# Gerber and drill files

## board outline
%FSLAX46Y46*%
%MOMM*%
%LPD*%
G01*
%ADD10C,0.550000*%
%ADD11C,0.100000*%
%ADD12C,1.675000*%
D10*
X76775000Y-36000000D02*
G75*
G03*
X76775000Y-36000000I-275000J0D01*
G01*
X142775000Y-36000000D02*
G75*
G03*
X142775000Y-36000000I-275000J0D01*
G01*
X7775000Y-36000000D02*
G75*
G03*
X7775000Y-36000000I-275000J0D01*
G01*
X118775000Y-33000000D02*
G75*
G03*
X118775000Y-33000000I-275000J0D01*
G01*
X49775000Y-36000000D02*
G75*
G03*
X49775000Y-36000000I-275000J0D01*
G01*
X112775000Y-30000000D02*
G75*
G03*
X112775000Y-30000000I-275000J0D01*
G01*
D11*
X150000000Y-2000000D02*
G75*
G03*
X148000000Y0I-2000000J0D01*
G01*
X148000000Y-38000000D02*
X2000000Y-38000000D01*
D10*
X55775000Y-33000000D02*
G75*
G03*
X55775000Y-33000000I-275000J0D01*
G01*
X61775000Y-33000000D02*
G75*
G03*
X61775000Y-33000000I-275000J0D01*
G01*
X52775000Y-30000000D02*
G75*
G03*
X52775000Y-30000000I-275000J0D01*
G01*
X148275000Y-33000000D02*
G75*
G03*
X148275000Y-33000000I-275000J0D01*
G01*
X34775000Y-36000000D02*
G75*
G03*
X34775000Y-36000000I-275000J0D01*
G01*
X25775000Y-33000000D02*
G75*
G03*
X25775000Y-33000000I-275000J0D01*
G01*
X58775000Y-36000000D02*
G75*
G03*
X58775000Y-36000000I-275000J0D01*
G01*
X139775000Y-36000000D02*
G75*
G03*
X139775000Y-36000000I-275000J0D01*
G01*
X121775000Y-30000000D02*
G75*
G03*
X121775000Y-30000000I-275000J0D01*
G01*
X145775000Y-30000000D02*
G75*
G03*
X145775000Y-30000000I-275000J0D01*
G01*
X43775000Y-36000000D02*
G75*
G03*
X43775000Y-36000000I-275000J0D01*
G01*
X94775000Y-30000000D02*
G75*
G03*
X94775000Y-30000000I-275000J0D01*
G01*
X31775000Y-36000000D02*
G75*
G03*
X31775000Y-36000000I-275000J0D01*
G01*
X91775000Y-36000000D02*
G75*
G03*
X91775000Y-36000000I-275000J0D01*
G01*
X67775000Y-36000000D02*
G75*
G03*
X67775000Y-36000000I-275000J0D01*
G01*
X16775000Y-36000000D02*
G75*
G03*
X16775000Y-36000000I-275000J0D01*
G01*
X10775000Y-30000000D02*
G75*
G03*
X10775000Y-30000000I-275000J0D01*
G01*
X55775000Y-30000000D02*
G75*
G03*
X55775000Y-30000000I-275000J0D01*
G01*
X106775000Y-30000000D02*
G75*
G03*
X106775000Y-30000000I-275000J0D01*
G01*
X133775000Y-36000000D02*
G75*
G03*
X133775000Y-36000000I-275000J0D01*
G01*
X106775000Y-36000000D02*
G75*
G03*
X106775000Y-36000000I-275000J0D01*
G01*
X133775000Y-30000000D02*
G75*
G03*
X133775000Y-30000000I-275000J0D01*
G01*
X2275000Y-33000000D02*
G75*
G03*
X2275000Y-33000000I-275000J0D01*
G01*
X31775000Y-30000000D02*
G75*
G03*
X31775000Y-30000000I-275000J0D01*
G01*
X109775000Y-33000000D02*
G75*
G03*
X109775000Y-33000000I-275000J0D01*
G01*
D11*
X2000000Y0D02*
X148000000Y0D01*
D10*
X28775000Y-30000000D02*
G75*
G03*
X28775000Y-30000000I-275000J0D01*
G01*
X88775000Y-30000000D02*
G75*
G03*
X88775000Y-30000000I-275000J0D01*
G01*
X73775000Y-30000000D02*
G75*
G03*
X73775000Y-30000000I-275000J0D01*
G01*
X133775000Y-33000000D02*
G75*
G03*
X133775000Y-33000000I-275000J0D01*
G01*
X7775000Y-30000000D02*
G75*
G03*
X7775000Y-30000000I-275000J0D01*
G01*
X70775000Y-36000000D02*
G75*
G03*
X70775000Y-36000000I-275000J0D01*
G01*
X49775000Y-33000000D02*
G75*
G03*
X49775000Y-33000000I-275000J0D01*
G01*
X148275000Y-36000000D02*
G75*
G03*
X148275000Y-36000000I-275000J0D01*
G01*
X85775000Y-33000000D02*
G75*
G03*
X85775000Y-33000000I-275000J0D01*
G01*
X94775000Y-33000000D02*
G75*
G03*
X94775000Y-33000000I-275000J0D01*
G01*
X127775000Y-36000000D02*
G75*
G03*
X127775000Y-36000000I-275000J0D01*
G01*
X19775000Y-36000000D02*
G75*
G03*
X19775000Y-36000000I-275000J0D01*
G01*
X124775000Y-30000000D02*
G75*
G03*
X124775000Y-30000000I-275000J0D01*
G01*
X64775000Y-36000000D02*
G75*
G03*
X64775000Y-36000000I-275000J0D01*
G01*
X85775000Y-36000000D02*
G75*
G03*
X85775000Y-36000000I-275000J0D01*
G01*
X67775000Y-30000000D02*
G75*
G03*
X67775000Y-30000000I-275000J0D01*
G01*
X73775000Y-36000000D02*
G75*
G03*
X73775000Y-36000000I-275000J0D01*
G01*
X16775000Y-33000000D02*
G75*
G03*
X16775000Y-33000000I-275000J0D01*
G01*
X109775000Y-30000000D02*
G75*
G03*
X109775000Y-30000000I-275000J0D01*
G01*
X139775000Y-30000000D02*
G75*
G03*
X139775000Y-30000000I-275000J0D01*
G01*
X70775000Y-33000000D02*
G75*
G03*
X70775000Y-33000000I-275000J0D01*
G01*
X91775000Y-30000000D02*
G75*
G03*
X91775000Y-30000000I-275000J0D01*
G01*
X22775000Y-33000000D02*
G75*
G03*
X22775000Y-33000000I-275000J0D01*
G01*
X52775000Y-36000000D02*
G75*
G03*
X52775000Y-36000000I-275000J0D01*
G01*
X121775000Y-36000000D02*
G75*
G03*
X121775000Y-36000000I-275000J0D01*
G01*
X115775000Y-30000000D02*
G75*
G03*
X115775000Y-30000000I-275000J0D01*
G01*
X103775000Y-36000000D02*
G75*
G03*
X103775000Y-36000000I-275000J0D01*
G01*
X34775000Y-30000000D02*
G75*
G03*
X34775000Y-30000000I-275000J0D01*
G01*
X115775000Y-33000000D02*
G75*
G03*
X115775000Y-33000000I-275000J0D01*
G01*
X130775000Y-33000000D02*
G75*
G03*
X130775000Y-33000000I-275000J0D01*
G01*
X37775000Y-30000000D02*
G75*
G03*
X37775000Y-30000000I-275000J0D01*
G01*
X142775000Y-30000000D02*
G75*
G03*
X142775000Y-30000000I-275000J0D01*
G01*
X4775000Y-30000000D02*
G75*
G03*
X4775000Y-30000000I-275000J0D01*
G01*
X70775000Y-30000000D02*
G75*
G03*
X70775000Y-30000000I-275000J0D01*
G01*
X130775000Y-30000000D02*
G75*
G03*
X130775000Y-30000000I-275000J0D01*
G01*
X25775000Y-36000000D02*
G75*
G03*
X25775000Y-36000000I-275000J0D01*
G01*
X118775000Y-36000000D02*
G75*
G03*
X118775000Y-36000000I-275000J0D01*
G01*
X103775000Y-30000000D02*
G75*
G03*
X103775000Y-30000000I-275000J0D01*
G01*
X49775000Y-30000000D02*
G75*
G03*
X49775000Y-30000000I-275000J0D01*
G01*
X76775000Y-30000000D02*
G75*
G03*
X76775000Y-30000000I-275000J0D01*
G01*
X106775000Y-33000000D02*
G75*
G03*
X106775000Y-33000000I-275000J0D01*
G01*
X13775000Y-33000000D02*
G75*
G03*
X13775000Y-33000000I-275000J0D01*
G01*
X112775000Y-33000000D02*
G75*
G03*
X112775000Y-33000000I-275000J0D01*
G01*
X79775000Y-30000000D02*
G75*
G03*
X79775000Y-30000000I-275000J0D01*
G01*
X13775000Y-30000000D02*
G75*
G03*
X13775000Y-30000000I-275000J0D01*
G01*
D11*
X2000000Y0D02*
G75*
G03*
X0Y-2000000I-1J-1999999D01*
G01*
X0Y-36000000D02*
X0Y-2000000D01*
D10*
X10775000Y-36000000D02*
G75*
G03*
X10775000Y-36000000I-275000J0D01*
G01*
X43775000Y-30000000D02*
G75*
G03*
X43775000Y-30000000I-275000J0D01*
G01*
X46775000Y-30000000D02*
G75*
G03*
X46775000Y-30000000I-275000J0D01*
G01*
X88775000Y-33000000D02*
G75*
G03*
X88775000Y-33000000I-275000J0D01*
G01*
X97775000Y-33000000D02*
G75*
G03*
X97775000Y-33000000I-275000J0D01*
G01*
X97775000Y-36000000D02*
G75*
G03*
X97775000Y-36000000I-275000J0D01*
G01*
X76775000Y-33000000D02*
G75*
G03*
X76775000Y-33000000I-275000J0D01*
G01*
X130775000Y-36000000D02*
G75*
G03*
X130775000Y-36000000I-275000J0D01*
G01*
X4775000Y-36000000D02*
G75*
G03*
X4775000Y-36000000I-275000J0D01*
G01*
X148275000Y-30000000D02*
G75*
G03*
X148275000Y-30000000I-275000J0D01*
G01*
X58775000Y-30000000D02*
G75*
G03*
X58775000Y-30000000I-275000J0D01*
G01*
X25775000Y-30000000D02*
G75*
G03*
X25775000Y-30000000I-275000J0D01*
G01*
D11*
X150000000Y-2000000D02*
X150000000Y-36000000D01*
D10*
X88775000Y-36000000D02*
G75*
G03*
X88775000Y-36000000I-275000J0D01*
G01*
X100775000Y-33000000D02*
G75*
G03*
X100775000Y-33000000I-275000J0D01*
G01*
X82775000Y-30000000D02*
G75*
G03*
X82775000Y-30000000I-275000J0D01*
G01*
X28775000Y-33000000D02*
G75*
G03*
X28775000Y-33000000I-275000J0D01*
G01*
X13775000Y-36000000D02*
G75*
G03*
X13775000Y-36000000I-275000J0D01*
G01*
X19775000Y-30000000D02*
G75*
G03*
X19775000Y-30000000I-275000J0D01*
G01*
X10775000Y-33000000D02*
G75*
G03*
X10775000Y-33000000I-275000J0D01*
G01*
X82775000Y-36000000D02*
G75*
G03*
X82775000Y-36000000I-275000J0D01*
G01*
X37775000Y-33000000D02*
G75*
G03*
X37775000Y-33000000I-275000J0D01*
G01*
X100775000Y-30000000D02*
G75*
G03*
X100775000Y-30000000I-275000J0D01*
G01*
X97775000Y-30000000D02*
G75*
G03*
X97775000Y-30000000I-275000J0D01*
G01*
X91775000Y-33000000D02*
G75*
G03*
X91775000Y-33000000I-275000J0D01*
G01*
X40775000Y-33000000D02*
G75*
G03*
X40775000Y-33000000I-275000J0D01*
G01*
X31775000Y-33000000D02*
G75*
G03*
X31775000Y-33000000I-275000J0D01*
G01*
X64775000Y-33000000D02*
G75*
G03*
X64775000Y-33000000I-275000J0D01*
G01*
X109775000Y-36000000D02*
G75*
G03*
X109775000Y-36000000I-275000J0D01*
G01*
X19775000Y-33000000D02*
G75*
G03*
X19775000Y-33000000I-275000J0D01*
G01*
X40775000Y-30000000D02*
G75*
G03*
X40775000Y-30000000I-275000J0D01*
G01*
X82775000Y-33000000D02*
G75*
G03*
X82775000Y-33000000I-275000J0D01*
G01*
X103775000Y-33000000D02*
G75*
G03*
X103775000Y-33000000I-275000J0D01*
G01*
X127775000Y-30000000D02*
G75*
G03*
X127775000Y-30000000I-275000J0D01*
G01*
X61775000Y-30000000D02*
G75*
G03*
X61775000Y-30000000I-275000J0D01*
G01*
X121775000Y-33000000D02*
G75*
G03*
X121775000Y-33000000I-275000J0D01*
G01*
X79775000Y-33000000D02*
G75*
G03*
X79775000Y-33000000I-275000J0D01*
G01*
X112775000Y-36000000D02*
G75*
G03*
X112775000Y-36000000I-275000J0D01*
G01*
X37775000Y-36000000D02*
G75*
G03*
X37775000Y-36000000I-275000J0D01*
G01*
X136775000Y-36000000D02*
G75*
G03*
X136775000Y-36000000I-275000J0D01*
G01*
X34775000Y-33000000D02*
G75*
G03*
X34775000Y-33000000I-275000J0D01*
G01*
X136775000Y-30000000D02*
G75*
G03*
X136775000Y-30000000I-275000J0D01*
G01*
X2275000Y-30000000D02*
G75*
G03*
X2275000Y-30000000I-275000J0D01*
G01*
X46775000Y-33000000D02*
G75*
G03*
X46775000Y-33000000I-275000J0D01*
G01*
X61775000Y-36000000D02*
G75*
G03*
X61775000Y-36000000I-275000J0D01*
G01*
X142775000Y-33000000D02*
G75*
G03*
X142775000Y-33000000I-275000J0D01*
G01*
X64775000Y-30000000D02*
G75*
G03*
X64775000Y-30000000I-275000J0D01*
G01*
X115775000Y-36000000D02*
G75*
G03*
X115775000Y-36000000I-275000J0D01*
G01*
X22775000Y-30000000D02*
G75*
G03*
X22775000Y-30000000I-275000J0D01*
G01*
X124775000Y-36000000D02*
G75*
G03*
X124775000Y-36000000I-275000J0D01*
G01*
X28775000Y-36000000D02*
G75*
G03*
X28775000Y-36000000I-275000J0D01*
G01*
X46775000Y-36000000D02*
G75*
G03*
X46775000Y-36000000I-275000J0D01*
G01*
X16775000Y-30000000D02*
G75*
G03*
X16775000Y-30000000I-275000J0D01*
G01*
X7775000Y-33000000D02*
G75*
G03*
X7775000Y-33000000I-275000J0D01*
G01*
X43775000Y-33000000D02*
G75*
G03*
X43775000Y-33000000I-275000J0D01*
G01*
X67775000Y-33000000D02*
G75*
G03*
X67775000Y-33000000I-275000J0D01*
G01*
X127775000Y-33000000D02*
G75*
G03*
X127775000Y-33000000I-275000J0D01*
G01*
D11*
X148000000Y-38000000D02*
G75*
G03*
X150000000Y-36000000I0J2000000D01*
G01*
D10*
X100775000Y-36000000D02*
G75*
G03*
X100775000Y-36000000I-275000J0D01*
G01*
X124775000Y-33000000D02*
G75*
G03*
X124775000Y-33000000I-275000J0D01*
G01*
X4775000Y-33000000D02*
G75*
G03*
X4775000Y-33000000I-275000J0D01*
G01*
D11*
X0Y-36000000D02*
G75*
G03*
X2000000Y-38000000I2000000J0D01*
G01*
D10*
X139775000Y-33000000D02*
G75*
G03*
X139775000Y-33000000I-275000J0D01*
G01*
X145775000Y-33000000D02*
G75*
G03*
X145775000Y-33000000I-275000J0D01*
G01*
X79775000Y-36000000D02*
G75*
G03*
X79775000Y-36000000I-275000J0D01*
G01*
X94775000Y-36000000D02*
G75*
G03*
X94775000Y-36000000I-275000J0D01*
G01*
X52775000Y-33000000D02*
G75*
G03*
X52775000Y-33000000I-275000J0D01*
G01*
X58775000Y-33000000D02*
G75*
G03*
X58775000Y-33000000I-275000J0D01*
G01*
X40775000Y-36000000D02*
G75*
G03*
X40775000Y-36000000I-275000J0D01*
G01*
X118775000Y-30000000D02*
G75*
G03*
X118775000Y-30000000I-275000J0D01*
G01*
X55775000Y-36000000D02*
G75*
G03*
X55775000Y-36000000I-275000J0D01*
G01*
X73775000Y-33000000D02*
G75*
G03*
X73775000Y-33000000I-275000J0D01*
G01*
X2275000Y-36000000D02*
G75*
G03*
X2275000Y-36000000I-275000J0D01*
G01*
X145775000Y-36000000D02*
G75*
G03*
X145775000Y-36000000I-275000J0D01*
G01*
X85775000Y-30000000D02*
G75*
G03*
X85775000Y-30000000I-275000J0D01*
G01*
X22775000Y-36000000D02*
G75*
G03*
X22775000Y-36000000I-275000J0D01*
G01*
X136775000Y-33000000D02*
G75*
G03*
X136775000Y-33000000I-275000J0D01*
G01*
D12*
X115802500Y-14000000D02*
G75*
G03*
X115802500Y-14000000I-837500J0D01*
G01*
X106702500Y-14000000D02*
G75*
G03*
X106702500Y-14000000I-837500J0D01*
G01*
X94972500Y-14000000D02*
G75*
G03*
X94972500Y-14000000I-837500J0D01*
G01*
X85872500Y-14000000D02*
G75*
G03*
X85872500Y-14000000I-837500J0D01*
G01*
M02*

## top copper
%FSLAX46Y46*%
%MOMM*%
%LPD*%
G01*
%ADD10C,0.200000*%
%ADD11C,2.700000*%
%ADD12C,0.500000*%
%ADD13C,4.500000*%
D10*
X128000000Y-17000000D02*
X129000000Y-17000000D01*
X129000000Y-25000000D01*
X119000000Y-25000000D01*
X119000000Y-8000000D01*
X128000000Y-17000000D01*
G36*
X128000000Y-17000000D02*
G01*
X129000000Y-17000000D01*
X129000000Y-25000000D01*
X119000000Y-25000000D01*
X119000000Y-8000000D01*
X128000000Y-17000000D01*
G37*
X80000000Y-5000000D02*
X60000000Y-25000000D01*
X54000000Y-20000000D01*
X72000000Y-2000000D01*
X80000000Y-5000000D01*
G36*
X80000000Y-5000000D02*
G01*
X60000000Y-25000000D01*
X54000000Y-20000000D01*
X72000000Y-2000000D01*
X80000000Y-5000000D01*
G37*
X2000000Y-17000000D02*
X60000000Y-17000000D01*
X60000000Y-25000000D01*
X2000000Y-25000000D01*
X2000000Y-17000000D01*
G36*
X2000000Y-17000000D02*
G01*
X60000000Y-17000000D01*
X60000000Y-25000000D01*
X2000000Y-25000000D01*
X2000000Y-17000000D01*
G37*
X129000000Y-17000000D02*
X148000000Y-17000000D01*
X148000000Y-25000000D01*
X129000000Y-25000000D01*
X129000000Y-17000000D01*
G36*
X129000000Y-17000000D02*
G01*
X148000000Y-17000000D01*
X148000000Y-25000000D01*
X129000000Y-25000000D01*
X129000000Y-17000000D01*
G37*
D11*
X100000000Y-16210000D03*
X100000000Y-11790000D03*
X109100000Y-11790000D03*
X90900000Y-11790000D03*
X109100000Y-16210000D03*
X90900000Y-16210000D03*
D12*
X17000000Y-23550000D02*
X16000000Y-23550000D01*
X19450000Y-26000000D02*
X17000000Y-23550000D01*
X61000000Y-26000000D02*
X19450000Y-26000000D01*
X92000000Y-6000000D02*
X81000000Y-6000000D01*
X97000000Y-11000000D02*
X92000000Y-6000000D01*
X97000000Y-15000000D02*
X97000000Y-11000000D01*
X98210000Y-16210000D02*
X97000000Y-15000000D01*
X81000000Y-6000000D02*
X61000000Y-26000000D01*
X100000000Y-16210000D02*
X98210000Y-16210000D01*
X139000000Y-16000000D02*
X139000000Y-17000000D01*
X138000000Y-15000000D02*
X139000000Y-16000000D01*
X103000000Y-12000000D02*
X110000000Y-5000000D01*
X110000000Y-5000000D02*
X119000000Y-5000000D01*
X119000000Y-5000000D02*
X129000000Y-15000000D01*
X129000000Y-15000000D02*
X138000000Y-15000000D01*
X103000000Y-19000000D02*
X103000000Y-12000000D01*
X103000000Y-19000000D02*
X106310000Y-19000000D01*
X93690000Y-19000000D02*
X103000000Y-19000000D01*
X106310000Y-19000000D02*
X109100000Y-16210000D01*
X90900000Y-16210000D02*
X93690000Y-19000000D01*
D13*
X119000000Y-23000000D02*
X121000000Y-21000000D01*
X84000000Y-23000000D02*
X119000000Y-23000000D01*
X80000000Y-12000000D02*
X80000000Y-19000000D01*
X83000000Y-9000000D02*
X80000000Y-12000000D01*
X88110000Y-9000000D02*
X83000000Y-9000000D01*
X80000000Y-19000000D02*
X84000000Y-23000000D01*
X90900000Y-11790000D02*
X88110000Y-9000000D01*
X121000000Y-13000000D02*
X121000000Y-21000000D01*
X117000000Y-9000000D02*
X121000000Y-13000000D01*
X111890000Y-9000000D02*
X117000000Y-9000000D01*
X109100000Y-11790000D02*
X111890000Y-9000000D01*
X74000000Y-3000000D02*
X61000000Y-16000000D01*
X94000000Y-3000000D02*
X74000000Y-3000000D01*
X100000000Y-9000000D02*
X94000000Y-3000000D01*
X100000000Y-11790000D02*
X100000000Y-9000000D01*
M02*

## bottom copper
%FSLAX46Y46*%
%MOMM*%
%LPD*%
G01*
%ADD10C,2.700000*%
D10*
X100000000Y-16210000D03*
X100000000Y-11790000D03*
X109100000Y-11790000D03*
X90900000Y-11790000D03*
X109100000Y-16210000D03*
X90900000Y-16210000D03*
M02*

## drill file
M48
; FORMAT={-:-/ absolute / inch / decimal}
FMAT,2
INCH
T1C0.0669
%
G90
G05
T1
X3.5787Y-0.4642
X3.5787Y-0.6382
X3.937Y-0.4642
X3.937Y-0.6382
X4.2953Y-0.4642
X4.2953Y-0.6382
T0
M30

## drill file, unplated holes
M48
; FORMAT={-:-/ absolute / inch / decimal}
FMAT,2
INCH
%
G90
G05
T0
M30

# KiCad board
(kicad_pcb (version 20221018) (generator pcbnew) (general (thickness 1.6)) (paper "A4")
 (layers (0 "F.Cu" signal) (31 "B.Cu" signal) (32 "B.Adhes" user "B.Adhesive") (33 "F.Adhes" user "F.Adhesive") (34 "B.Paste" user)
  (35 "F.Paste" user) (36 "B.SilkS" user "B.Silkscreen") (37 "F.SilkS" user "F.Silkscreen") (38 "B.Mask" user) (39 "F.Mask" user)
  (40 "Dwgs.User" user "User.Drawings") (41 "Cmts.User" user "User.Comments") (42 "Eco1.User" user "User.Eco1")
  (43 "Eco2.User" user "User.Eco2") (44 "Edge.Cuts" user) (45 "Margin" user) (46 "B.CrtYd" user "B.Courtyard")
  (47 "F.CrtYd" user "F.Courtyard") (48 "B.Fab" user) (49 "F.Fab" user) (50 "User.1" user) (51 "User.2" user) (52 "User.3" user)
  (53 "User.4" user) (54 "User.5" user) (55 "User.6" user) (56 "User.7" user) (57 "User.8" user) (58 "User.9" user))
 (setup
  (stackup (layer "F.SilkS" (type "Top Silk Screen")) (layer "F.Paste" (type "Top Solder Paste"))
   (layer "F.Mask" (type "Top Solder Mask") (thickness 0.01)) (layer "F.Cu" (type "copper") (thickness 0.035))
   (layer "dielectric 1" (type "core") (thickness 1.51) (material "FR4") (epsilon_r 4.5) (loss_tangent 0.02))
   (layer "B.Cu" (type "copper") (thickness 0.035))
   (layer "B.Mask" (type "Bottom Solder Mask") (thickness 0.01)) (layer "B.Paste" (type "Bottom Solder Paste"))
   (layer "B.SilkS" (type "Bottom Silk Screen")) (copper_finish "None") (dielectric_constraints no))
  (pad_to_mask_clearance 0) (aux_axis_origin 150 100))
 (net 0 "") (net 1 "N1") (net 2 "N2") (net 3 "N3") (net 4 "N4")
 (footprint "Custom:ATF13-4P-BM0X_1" (layer "F.Cu") (at 100 14 180)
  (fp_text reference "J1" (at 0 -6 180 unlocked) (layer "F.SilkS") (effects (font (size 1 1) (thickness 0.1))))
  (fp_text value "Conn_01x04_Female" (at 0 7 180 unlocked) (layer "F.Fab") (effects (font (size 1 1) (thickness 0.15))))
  (fp_circle (center -14.965 0) (end -13.315 0) (stroke (width 0.05) (type solid)) (fill solid) (layer "Edge.Cuts"))
  (fp_circle (center -5.865 0) (end -4.215 0) (stroke (width 0.05) (type solid)) (fill solid) (layer "Edge.Cuts"))
  (fp_circle (center 5.865 0) (end 7.515 0) (stroke (width 0.05) (type solid)) (fill solid) (layer "Edge.Cuts"))
  (fp_circle (center 14.965 0) (end 16.615 0) (stroke (width 0.05) (type solid)) (fill solid) (layer "Edge.Cuts"))
  (pad "1" thru_hole circle (at 0 -2.21 180) (size 2.7 2.7) (drill 1.7) (layers "*.Cu" "*.Mask") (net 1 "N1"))
  (pad "2" thru_hole circle (at 0 2.21 180) (size 2.7 2.7) (drill 1.7) (layers "*.Cu" "*.Mask") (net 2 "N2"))
  (pad "3" thru_hole circle (at -9.1 2.21 180) (size 2.7 2.7) (drill 1.7) (layers "*.Cu" "*.Mask") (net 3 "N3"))
  (pad "3" thru_hole circle (at 9.1 2.21 180) (size 2.7 2.7) (drill 1.7) (layers "*.Cu" "*.Mask") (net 3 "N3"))
  (pad "4" thru_hole circle (at -9.1 -2.21 180) (size 2.7 2.7) (drill 1.7) (layers "*.Cu" "*.Mask") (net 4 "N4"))
  (pad "4" thru_hole circle (at 9.1 -2.21 180) (size 2.7 2.7) (drill 1.7) (layers "*.Cu" "*.Mask") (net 4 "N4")))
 (gr_poly (pts (xy 60 25) (xy 80 5) (xy 72 2) (xy 54 20)) (stroke (width 0.2) (type solid)) (fill solid) (layer "F.Cu"))
 (gr_poly (pts (xy 129 25) (xy 119 25) (xy 119 8) (xy 128 17) (xy 129 17)) (stroke (width 0.2) (type solid)) (fill solid) (layer "F.Cu"))
 (gr_rect (start 2 17) (end 60 25) (stroke (width 0.2) (type solid)) (fill solid) (layer "F.Cu"))
 (gr_rect (start 129 17) (end 148 25) (stroke (width 0.2) (type solid)) (fill solid) (layer "F.Cu"))
 (gr_circle (center 76.5 36) (end 76.5 36.5) (stroke (width 0.1) (type solid)) (fill solid) (layer "Edge.Cuts"))
 (gr_circle (center 142.5 36) (end 142.5 36.5) (stroke (width 0.1) (type solid)) (fill solid) (layer "Edge.Cuts"))
 (gr_circle (center 7.5 36) (end 7.5 36.5) (stroke (width 0.1) (type solid)) (fill solid) (layer "Edge.Cuts"))
 (gr_circle (center 118.5 33) (end 118.5 33.5) (stroke (width 0.1) (type solid)) (fill solid) (layer "Edge.Cuts"))
 (gr_circle (center 49.5 36) (end 49.5 36.5) (stroke (width 0.1) (type solid)) (fill solid) (layer "Edge.Cuts"))
 (gr_circle (center 112.5 30) (end 112.5 30.5) (stroke (width 0.1) (type solid)) (fill solid) (layer "Edge.Cuts"))
 (gr_arc (start 148 0) (mid 149.414214 0.585786) (end 150 2) (stroke (width 0.1) (type default)) (layer "Edge.Cuts"))
 (gr_line (start 148 38) (end 2 38) (stroke (width 0.1) (type default)) (layer "Edge.Cuts"))
 (gr_circle (center 55.5 33) (end 55.5 33.5) (stroke (width 0.1) (type solid)) (fill solid) (layer "Edge.Cuts"))
 (gr_circle (center 61.5 33) (end 61.5 33.5) (stroke (width 0.1) (type solid)) (fill solid) (layer "Edge.Cuts"))
 (gr_circle (center 52.5 30) (end 52.5 30.5) (stroke (width 0.1) (type solid)) (fill solid) (layer "Edge.Cuts"))
 (gr_circle (center 148 33) (end 148 33.5) (stroke (width 0.1) (type solid)) (fill solid) (layer "Edge.Cuts"))
 (gr_circle (center 34.5 36) (end 34.5 36.5) (stroke (width 0.1) (type solid)) (fill solid) (layer "Edge.Cuts"))
 (gr_circle (center 25.5 33) (end 25.5 33.5) (stroke (width 0.1) (type solid)) (fill solid) (layer "Edge.Cuts"))
 (gr_circle (center 58.5 36) (end 58.5 36.5) (stroke (width 0.1) (type solid)) (fill solid) (layer "Edge.Cuts"))
 (gr_circle (center 139.5 36) (end 139.5 36.5) (stroke (width 0.1) (type solid)) (fill solid) (layer "Edge.Cuts"))
 (gr_circle (center 121.5 30) (end 121.5 30.5) (stroke (width 0.1) (type solid)) (fill solid) (layer "Edge.Cuts"))
 (gr_circle (center 145.5 30) (end 145.5 30.5) (stroke (width 0.1) (type solid)) (fill solid) (layer "Edge.Cuts"))
 (gr_circle (center 43.5 36) (end 43.5 36.5) (stroke (width 0.1) (type solid)) (fill solid) (layer "Edge.Cuts"))
 (gr_circle (center 94.5 30) (end 94.5 30.5) (stroke (width 0.1) (type solid)) (fill solid) (layer "Edge.Cuts"))
 (gr_circle (center 31.5 36) (end 31.5 36.5) (stroke (width 0.1) (type solid)) (fill solid) (layer "Edge.Cuts"))
 (gr_circle (center 91.5 36) (end 91.5 36.5) (stroke (width 0.1) (type solid)) (fill solid) (layer "Edge.Cuts"))
 (gr_circle (center 67.5 36) (end 67.5 36.5) (stroke (width 0.1) (type solid)) (fill solid) (layer "Edge.Cuts"))
 (gr_circle (center 16.5 36) (end 16.5 36.5) (stroke (width 0.1) (type solid)) (fill solid) (layer "Edge.Cuts"))
 (gr_circle (center 10.5 30) (end 10.5 30.5) (stroke (width 0.1) (type solid)) (fill solid) (layer "Edge.Cuts"))
 (gr_circle (center 55.5 30) (end 55.5 30.5) (stroke (width 0.1) (type solid)) (fill solid) (layer "Edge.Cuts"))
 (gr_circle (center 106.5 30) (end 106.5 30.5) (stroke (width 0.1) (type solid)) (fill solid) (layer "Edge.Cuts"))
 (gr_circle (center 133.5 36) (end 133.5 36.5) (stroke (width 0.1) (type solid)) (fill solid) (layer "Edge.Cuts"))
 (gr_circle (center 106.5 36) (end 106.5 36.5) (stroke (width 0.1) (type solid)) (fill solid) (layer "Edge.Cuts"))
 (gr_circle (center 133.5 30) (end 133.5 30.5) (stroke (width 0.1) (type solid)) (fill solid) (layer "Edge.Cuts"))
 (gr_circle (center 2 33) (end 2 33.5) (stroke (width 0.1) (type solid)) (fill solid) (layer "Edge.Cuts"))
 (gr_circle (center 31.5 30) (end 31.5 30.5) (stroke (width 0.1) (type solid)) (fill solid) (layer "Edge.Cuts"))
 (gr_circle (center 109.5 33) (end 109.5 33.5) (stroke (width 0.1) (type solid)) (fill solid) (layer "Edge.Cuts"))
 (gr_line (start 2 0) (end 148 0) (stroke (width 0.1) (type default)) (layer "Edge.Cuts"))
 (gr_circle (center 28.5 30) (end 28.5 30.5) (stroke (width 0.1) (type solid)) (fill solid) (layer "Edge.Cuts"))
 (gr_circle (center 88.5 30) (end 88.5 30.5) (stroke (width 0.1) (type solid)) (fill solid) (layer "Edge.Cuts"))
 (gr_circle (center 73.5 30) (end 73.5 30.5) (stroke (width 0.1) (type solid)) (fill solid) (layer "Edge.Cuts"))
 (gr_circle (center 133.5 33) (end 133.5 33.5) (stroke (width 0.1) (type solid)) (fill solid) (layer "Edge.Cuts"))
 (gr_circle (center 7.5 30) (end 7.5 30.5) (stroke (width 0.1) (type solid)) (fill solid) (layer "Edge.Cuts"))
 (gr_circle (center 70.5 36) (end 70.5 36.5) (stroke (width 0.1) (type solid)) (fill solid) (layer "Edge.Cuts"))
 (gr_circle (center 49.5 33) (end 49.5 33.5) (stroke (width 0.1) (type solid)) (fill solid) (layer "Edge.Cuts"))
 (gr_circle (center 148 36) (end 148 36.5) (stroke (width 0.1) (type solid)) (fill solid) (layer "Edge.Cuts"))
 (gr_circle (center 85.5 33) (end 85.5 33.5) (stroke (width 0.1) (type solid)) (fill solid) (layer "Edge.Cuts"))
 (gr_circle (center 94.5 33) (end 94.5 33.5) (stroke (width 0.1) (type solid)) (fill solid) (layer "Edge.Cuts"))
 (gr_circle (center 127.5 36) (end 127.5 36.5) (stroke (width 0.1) (type solid)) (fill solid) (layer "Edge.Cuts"))
 (gr_circle (center 19.5 36) (end 19.5 36.5) (stroke (width 0.1) (type solid)) (fill solid) (layer "Edge.Cuts"))
 (gr_circle (center 124.5 30) (end 124.5 30.5) (stroke (width 0.1) (type solid)) (fill solid) (layer "Edge.Cuts"))
 (gr_circle (center 64.5 36) (end 64.5 36.5) (stroke (width 0.1) (type solid)) (fill solid) (layer "Edge.Cuts"))
 (gr_circle (center 85.5 36) (end 85.5 36.5) (stroke (width 0.1) (type solid)) (fill solid) (layer "Edge.Cuts"))
 (gr_circle (center 67.5 30) (end 67.5 30.5) (stroke (width 0.1) (type solid)) (fill solid) (layer "Edge.Cuts"))
 (gr_circle (center 73.5 36) (end 73.5 36.5) (stroke (width 0.1) (type solid)) (fill solid) (layer "Edge.Cuts"))
 (gr_circle (center 16.5 33) (end 16.5 33.5) (stroke (width 0.1) (type solid)) (fill solid) (layer "Edge.Cuts"))
 (gr_circle (center 109.5 30) (end 109.5 30.5) (stroke (width 0.1) (type solid)) (fill solid) (layer "Edge.Cuts"))
 (gr_circle (center 139.5 30) (end 139.5 30.5) (stroke (width 0.1) (type solid)) (fill solid) (layer "Edge.Cuts"))
 (gr_circle (center 70.5 33) (end 70.5 33.5) (stroke (width 0.1) (type solid)) (fill solid) (layer "Edge.Cuts"))
 (gr_circle (center 91.5 30) (end 91.5 30.5) (stroke (width 0.1) (type solid)) (fill solid) (layer "Edge.Cuts"))
 (gr_circle (center 22.5 33) (end 22.5 33.5) (stroke (width 0.1) (type solid)) (fill solid) (layer "Edge.Cuts"))
 (gr_circle (center 52.5 36) (end 52.5 36.5) (stroke (width 0.1) (type solid)) (fill solid) (layer "Edge.Cuts"))
 (gr_circle (center 121.5 36) (end 121.5 36.5) (stroke (width 0.1) (type solid)) (fill solid) (layer "Edge.Cuts"))
 (gr_circle (center 115.5 30) (end 115.5 30.5) (stroke (width 0.1) (type solid)) (fill solid) (layer "Edge.Cuts"))
 (gr_circle (center 103.5 36) (end 103.5 36.5) (stroke (width 0.1) (type solid)) (fill solid) (layer "Edge.Cuts"))
 (gr_circle (center 34.5 30) (end 34.5 30.5) (stroke (width 0.1) (type solid)) (fill solid) (layer "Edge.Cuts"))
 (gr_circle (center 115.5 33) (end 115.5 33.5) (stroke (width 0.1) (type solid)) (fill solid) (layer "Edge.Cuts"))
 (gr_circle (center 130.5 33) (end 130.5 33.5) (stroke (width 0.1) (type solid)) (fill solid) (layer "Edge.Cuts"))
 (gr_circle (center 37.5 30) (end 37.5 30.5) (stroke (width 0.1) (type solid)) (fill solid) (layer "Edge.Cuts"))
 (gr_circle (center 142.5 30) (end 142.5 30.5) (stroke (width 0.1) (type solid)) (fill solid) (layer "Edge.Cuts"))
 (gr_circle (center 4.5 30) (end 4.5 30.5) (stroke (width 0.1) (type solid)) (fill solid) (layer "Edge.Cuts"))
 (gr_circle (center 70.5 30) (end 70.5 30.5) (stroke (width 0.1) (type solid)) (fill solid) (layer "Edge.Cuts"))
 (gr_circle (center 130.5 30) (end 130.5 30.5) (stroke (width 0.1) (type solid)) (fill solid) (layer "Edge.Cuts"))
 (gr_circle (center 25.5 36) (end 25.5 36.5) (stroke (width 0.1) (type solid)) (fill solid) (layer "Edge.Cuts"))
 (gr_circle (center 118.5 36) (end 118.5 36.5) (stroke (width 0.1) (type solid)) (fill solid) (layer "Edge.Cuts"))
 (gr_circle (center 103.5 30) (end 103.5 30.5) (stroke (width 0.1) (type solid)) (fill solid) (layer "Edge.Cuts"))
 (gr_circle (center 49.5 30) (end 49.5 30.5) (stroke (width 0.1) (type solid)) (fill solid) (layer "Edge.Cuts"))
 (gr_circle (center 76.5 30) (end 76.5 30.5) (stroke (width 0.1) (type solid)) (fill solid) (layer "Edge.Cuts"))
 (gr_circle (center 106.5 33) (end 106.5 33.5) (stroke (width 0.1) (type solid)) (fill solid) (layer "Edge.Cuts"))
 (gr_circle (center 13.5 33) (end 13.5 33.5) (stroke (width 0.1) (type solid)) (fill solid) (layer "Edge.Cuts"))
 (gr_circle (center 112.5 33) (end 112.5 33.5) (stroke (width 0.1) (type solid)) (fill solid) (layer "Edge.Cuts"))
 (gr_circle (center 79.5 30) (end 79.5 30.5) (stroke (width 0.1) (type solid)) (fill solid) (layer "Edge.Cuts"))
 (gr_circle (center 13.5 30) (end 13.5 30.5) (stroke (width 0.1) (type solid)) (fill solid) (layer "Edge.Cuts"))
 (gr_arc (start 0 2) (mid 0.585786 0.585786) (end 2 0) (stroke (width 0.1) (type default)) (layer "Edge.Cuts"))
 (gr_line (start 0 36) (end 0 2) (stroke (width 0.1) (type default)) (layer "Edge.Cuts"))
 (gr_circle (center 10.5 36) (end 10.5 36.5) (stroke (width 0.1) (type solid)) (fill solid) (layer "Edge.Cuts"))
 (gr_circle (center 43.5 30) (end 43.5 30.5) (stroke (width 0.1) (type solid)) (fill solid) (layer "Edge.Cuts"))
 (gr_circle (center 46.5 30) (end 46.5 30.5) (stroke (width 0.1) (type solid)) (fill solid) (layer "Edge.Cuts"))
 (gr_circle (center 88.5 33) (end 88.5 33.5) (stroke (width 0.1) (type solid)) (fill solid) (layer "Edge.Cuts"))
 (gr_circle (center 97.5 33) (end 97.5 33.5) (stroke (width 0.1) (type solid)) (fill solid) (layer "Edge.Cuts"))
 (gr_circle (center 97.5 36) (end 97.5 36.5) (stroke (width 0.1) (type solid)) (fill solid) (layer "Edge.Cuts"))
 (gr_circle (center 76.5 33) (end 76.5 33.5) (stroke (width 0.1) (type solid)) (fill solid) (layer "Edge.Cuts"))
 (gr_circle (center 130.5 36) (end 130.5 36.5) (stroke (width 0.1) (type solid)) (fill solid) (layer "Edge.Cuts"))
 (gr_circle (center 4.5 36) (end 4.5 36.5) (stroke (width 0.1) (type solid)) (fill solid) (layer "Edge.Cuts"))
 (gr_circle (center 148 30) (end 148 30.5) (stroke (width 0.1) (type solid)) (fill solid) (layer "Edge.Cuts"))
 (gr_circle (center 58.5 30) (end 58.5 30.5) (stroke (width 0.1) (type solid)) (fill solid) (layer "Edge.Cuts"))
 (gr_circle (center 25.5 30) (end 25.5 30.5) (stroke (width 0.1) (type solid)) (fill solid) (layer "Edge.Cuts"))
 (gr_line (start 150 2) (end 150 36) (stroke (width 0.1) (type default)) (layer "Edge.Cuts"))
 (gr_circle (center 88.5 36) (end 88.5 36.5) (stroke (width 0.1) (type solid)) (fill solid) (layer "Edge.Cuts"))
 (gr_circle (center 100.5 33) (end 100.5 33.5) (stroke (width 0.1) (type solid)) (fill solid) (layer "Edge.Cuts"))
 (gr_circle (center 82.5 30) (end 82.5 30.5) (stroke (width 0.1) (type solid)) (fill solid) (layer "Edge.Cuts"))
 (gr_circle (center 28.5 33) (end 28.5 33.5) (stroke (width 0.1) (type solid)) (fill solid) (layer "Edge.Cuts"))
 (gr_circle (center 13.5 36) (end 13.5 36.5) (stroke (width 0.1) (type solid)) (fill solid) (layer "Edge.Cuts"))
 (gr_circle (center 19.5 30) (end 19.5 30.5) (stroke (width 0.1) (type solid)) (fill solid) (layer "Edge.Cuts"))
 (gr_circle (center 10.5 33) (end 10.5 33.5) (stroke (width 0.1) (type solid)) (fill solid) (layer "Edge.Cuts"))
 (gr_circle (center 82.5 36) (end 82.5 36.5) (stroke (width 0.1) (type solid)) (fill solid) (layer "Edge.Cuts"))
 (gr_circle (center 37.5 33) (end 37.5 33.5) (stroke (width 0.1) (type solid)) (fill solid) (layer "Edge.Cuts"))
 (gr_circle (center 100.5 30) (end 100.5 30.5) (stroke (width 0.1) (type solid)) (fill solid) (layer "Edge.Cuts"))
 (gr_circle (center 97.5 30) (end 97.5 30.5) (stroke (width 0.1) (type solid)) (fill solid) (layer "Edge.Cuts"))
 (gr_circle (center 91.5 33) (end 91.5 33.5) (stroke (width 0.1) (type solid)) (fill solid) (layer "Edge.Cuts"))
 (gr_circle (center 40.5 33) (end 40.5 33.5) (stroke (width 0.1) (type solid)) (fill solid) (layer "Edge.Cuts"))
 (gr_circle (center 31.5 33) (end 31.5 33.5) (stroke (width 0.1) (type solid)) (fill solid) (layer "Edge.Cuts"))
 (gr_circle (center 64.5 33) (end 64.5 33.5) (stroke (width 0.1) (type solid)) (fill solid) (layer "Edge.Cuts"))
 (gr_circle (center 109.5 36) (end 109.5 36.5) (stroke (width 0.1) (type solid)) (fill solid) (layer "Edge.Cuts"))
 (gr_circle (center 19.5 33) (end 19.5 33.5) (stroke (width 0.1) (type solid)) (fill solid) (layer "Edge.Cuts"))
 (gr_circle (center 40.5 30) (end 40.5 30.5) (stroke (width 0.1) (type solid)) (fill solid) (layer "Edge.Cuts"))
 (gr_circle (center 82.5 33) (end 82.5 33.5) (stroke (width 0.1) (type solid)) (fill solid) (layer "Edge.Cuts"))
 (gr_circle (center 103.5 33) (end 103.5 33.5) (stroke (width 0.1) (type solid)) (fill solid) (layer "Edge.Cuts"))
 (gr_circle (center 127.5 30) (end 127.5 30.5) (stroke (width 0.1) (type solid)) (fill solid) (layer "Edge.Cuts"))
 (gr_circle (center 61.5 30) (end 61.5 30.5) (stroke (width 0.1) (type solid)) (fill solid) (layer "Edge.Cuts"))
 (gr_circle (center 121.5 33) (end 121.5 33.5) (stroke (width 0.1) (type solid)) (fill solid) (layer "Edge.Cuts"))
 (gr_circle (center 79.5 33) (end 79.5 33.5) (stroke (width 0.1) (type solid)) (fill solid) (layer "Edge.Cuts"))
 (gr_circle (center 112.5 36) (end 112.5 36.5) (stroke (width 0.1) (type solid)) (fill solid) (layer "Edge.Cuts"))
 (gr_circle (center 37.5 36) (end 37.5 36.5) (stroke (width 0.1) (type solid)) (fill solid) (layer "Edge.Cuts"))
 (gr_circle (center 136.5 36) (end 136.5 36.5) (stroke (width 0.1) (type solid)) (fill solid) (layer "Edge.Cuts"))
 (gr_circle (center 34.5 33) (end 34.5 33.5) (stroke (width 0.1) (type solid)) (fill solid) (layer "Edge.Cuts"))
 (gr_circle (center 136.5 30) (end 136.5 30.5) (stroke (width 0.1) (type solid)) (fill solid) (layer "Edge.Cuts"))
 (gr_circle (center 2 30) (end 2 30.5) (stroke (width 0.1) (type solid)) (fill solid) (layer "Edge.Cuts"))
 (gr_circle (center 46.5 33) (end 46.5 33.5) (stroke (width 0.1) (type solid)) (fill solid) (layer "Edge.Cuts"))
 (gr_circle (center 61.5 36) (end 61.5 36.5) (stroke (width 0.1) (type solid)) (fill solid) (layer "Edge.Cuts"))
 (gr_circle (center 142.5 33) (end 142.5 33.5) (stroke (width 0.1) (type solid)) (fill solid) (layer "Edge.Cuts"))
 (gr_circle (center 64.5 30) (end 64.5 30.5) (stroke (width 0.1) (type solid)) (fill solid) (layer "Edge.Cuts"))
 (gr_circle (center 115.5 36) (end 115.5 36.5) (stroke (width 0.1) (type solid)) (fill solid) (layer "Edge.Cuts"))
 (gr_circle (center 22.5 30) (end 22.5 30.5) (stroke (width 0.1) (type solid)) (fill solid) (layer "Edge.Cuts"))
 (gr_circle (center 124.5 36) (end 124.5 36.5) (stroke (width 0.1) (type solid)) (fill solid) (layer "Edge.Cuts"))
 (gr_circle (center 28.5 36) (end 28.5 36.5) (stroke (width 0.1) (type solid)) (fill solid) (layer "Edge.Cuts"))
 (gr_circle (center 46.5 36) (end 46.5 36.5) (stroke (width 0.1) (type solid)) (fill solid) (layer "Edge.Cuts"))
 (gr_circle (center 16.5 30) (end 16.5 30.5) (stroke (width 0.1) (type solid)) (fill solid) (layer "Edge.Cuts"))
 (gr_circle (center 7.5 33) (end 7.5 33.5) (stroke (width 0.1) (type solid)) (fill solid) (layer "Edge.Cuts"))
 (gr_circle (center 43.5 33) (end 43.5 33.5) (stroke (width 0.1) (type solid)) (fill solid) (layer "Edge.Cuts"))
 (gr_circle (center 67.5 33) (end 67.5 33.5) (stroke (width 0.1) (type solid)) (fill solid) (layer "Edge.Cuts"))
 (gr_circle (center 127.5 33) (end 127.5 33.5) (stroke (width 0.1) (type solid)) (fill solid) (layer "Edge.Cuts"))
 (gr_arc (start 150 36) (mid 149.414214 37.414214) (end 148 38) (stroke (width 0.1) (type default)) (layer "Edge.Cuts"))
 (gr_circle (center 100.5 36) (end 100.5 36.5) (stroke (width 0.1) (type solid)) (fill solid) (layer "Edge.Cuts"))
 (gr_circle (center 124.5 33) (end 124.5 33.5) (stroke (width 0.1) (type solid)) (fill solid) (layer "Edge.Cuts"))
 (gr_circle (center 4.5 33) (end 4.5 33.5) (stroke (width 0.1) (type solid)) (fill solid) (layer "Edge.Cuts"))
 (gr_arc (start 2 38) (mid 0.585786 37.414214) (end 0 36) (stroke (width 0.1) (type default)) (layer "Edge.Cuts"))
 (gr_circle (center 139.5 33) (end 139.5 33.5) (stroke (width 0.1) (type solid)) (fill solid) (layer "Edge.Cuts"))
 (gr_circle (center 145.5 33) (end 145.5 33.5) (stroke (width 0.1) (type solid)) (fill solid) (layer "Edge.Cuts"))
 (gr_circle (center 79.5 36) (end 79.5 36.5) (stroke (width 0.1) (type solid)) (fill solid) (layer "Edge.Cuts"))
 (gr_circle (center 94.5 36) (end 94.5 36.5) (stroke (width 0.1) (type solid)) (fill solid) (layer "Edge.Cuts"))
 (gr_circle (center 52.5 33) (end 52.5 33.5) (stroke (width 0.1) (type solid)) (fill solid) (layer "Edge.Cuts"))
 (gr_circle (center 58.5 33) (end 58.5 33.5) (stroke (width 0.1) (type solid)) (fill solid) (layer "Edge.Cuts"))
 (gr_circle (center 40.5 36) (end 40.5 36.5) (stroke (width 0.1) (type solid)) (fill solid) (layer "Edge.Cuts"))
 (gr_circle (center 118.5 30) (end 118.5 30.5) (stroke (width 0.1) (type solid)) (fill solid) (layer "Edge.Cuts"))
 (gr_circle (center 55.5 36) (end 55.5 36.5) (stroke (width 0.1) (type solid)) (fill solid) (layer "Edge.Cuts"))
 (gr_circle (center 73.5 33) (end 73.5 33.5) (stroke (width 0.1) (type solid)) (fill solid) (layer "Edge.Cuts"))
 (gr_circle (center 2 36) (end 2 36.5) (stroke (width 0.1) (type solid)) (fill solid) (layer "Edge.Cuts"))
 (gr_circle (center 145.5 36) (end 145.5 36.5) (stroke (width 0.1) (type solid)) (fill solid) (layer "Edge.Cuts"))
 (gr_circle (center 85.5 30) (end 85.5 30.5) (stroke (width 0.1) (type solid)) (fill solid) (layer "Edge.Cuts"))
 (gr_circle (center 22.5 36) (end 22.5 36.5) (stroke (width 0.1) (type solid)) (fill solid) (layer "Edge.Cuts"))
 (gr_circle (center 136.5 33) (end 136.5 33.5) (stroke (width 0.1) (type solid)) (fill solid) (layer "Edge.Cuts"))
 (segment (start 61 26) (end 19.45 26) (width 0.5) (layer "F.Cu") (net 1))
 (segment (start 81 6) (end 61 26) (width 0.5) (layer "F.Cu") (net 1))
 (segment (start 17 23.55) (end 16 23.55) (width 0.5) (layer "F.Cu") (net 1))
 (segment (start 97 11) (end 92 6) (width 0.5) (layer "F.Cu") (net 1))
 (segment (start 100 16.21) (end 98.21 16.21) (width 0.5) (layer "F.Cu") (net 1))
 (segment (start 97 15) (end 97 11) (width 0.5) (layer "F.Cu") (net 1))
 (segment (start 19.45 26) (end 17 23.55) (width 0.5) (layer "F.Cu") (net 1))
 (segment (start 98.21 16.21) (end 97 15) (width 0.5) (layer "F.Cu") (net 1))
 (segment (start 92 6) (end 81 6) (width 0.5) (layer "F.Cu") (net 1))
 (segment (start 100 11.79) (end 100 9) (width 4.5) (layer "F.Cu") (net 2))
 (segment (start 74 3) (end 61 16) (width 4.5) (layer "F.Cu") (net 2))
 (segment (start 94 3) (end 74 3) (width 4.5) (layer "F.Cu") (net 2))
 (segment (start 100 9) (end 94 3) (width 4.5) (layer "F.Cu") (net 2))
 (segment (start 111.89 9) (end 117 9) (width 4.5) (layer "F.Cu") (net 3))
 (segment (start 119 23) (end 121 21) (width 4.5) (layer "F.Cu") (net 3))
 (segment (start 84 23) (end 119 23) (width 4.5) (layer "F.Cu") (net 3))
 (segment (start 109.1 11.79) (end 111.89 9) (width 4.5) (layer "F.Cu") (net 3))
 (segment (start 80 12) (end 80 19) (width 4.5) (layer "F.Cu") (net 3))
 (segment (start 117 9) (end 121 13) (width 4.5) (layer "F.Cu") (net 3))
 (segment (start 80 19) (end 84 23) (width 4.5) (layer "F.Cu") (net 3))
 (segment (start 121 13) (end 121 21) (width 4.5) (layer "F.Cu") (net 3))
 (segment (start 90.9 11.79) (end 88.11 9) (width 4.5) (layer "F.Cu") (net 3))
 (segment (start 88.11 9) (end 83 9) (width 4.5) (layer "F.Cu") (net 3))
 (segment (start 83 9) (end 80 12) (width 4.5) (layer "F.Cu") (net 3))
 (segment (start 110 5) (end 119 5) (width 0.5) (layer "F.Cu") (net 4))
 (segment (start 90.9 16.21) (end 93.69 19) (width 0.5) (layer "F.Cu") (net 4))
 (segment (start 103 12) (end 110 5) (width 0.5) (layer "F.Cu") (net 4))
 (segment (start 138 15) (end 139 16) (width 0.5) (layer "F.Cu") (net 4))
 (segment (start 93.69 19) (end 103 19) (width 0.5) (layer "F.Cu") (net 4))
 (segment (start 103 19) (end 106.31 19) (width 0.5) (layer "F.Cu") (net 4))
 (segment (start 119 5) (end 129 15) (width 0.5) (layer "F.Cu") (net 4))
 (segment (start 139 16) (end 139 17) (width 0.5) (layer "F.Cu") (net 4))
 (segment (start 103 19) (end 103 12) (width 0.5) (layer "F.Cu") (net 4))
 (segment (start 129 15) (end 138 15) (width 0.5) (layer "F.Cu") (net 4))
 (segment (start 106.31 19) (end 109.1 16.21) (width 0.5) (layer "F.Cu") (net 4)))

